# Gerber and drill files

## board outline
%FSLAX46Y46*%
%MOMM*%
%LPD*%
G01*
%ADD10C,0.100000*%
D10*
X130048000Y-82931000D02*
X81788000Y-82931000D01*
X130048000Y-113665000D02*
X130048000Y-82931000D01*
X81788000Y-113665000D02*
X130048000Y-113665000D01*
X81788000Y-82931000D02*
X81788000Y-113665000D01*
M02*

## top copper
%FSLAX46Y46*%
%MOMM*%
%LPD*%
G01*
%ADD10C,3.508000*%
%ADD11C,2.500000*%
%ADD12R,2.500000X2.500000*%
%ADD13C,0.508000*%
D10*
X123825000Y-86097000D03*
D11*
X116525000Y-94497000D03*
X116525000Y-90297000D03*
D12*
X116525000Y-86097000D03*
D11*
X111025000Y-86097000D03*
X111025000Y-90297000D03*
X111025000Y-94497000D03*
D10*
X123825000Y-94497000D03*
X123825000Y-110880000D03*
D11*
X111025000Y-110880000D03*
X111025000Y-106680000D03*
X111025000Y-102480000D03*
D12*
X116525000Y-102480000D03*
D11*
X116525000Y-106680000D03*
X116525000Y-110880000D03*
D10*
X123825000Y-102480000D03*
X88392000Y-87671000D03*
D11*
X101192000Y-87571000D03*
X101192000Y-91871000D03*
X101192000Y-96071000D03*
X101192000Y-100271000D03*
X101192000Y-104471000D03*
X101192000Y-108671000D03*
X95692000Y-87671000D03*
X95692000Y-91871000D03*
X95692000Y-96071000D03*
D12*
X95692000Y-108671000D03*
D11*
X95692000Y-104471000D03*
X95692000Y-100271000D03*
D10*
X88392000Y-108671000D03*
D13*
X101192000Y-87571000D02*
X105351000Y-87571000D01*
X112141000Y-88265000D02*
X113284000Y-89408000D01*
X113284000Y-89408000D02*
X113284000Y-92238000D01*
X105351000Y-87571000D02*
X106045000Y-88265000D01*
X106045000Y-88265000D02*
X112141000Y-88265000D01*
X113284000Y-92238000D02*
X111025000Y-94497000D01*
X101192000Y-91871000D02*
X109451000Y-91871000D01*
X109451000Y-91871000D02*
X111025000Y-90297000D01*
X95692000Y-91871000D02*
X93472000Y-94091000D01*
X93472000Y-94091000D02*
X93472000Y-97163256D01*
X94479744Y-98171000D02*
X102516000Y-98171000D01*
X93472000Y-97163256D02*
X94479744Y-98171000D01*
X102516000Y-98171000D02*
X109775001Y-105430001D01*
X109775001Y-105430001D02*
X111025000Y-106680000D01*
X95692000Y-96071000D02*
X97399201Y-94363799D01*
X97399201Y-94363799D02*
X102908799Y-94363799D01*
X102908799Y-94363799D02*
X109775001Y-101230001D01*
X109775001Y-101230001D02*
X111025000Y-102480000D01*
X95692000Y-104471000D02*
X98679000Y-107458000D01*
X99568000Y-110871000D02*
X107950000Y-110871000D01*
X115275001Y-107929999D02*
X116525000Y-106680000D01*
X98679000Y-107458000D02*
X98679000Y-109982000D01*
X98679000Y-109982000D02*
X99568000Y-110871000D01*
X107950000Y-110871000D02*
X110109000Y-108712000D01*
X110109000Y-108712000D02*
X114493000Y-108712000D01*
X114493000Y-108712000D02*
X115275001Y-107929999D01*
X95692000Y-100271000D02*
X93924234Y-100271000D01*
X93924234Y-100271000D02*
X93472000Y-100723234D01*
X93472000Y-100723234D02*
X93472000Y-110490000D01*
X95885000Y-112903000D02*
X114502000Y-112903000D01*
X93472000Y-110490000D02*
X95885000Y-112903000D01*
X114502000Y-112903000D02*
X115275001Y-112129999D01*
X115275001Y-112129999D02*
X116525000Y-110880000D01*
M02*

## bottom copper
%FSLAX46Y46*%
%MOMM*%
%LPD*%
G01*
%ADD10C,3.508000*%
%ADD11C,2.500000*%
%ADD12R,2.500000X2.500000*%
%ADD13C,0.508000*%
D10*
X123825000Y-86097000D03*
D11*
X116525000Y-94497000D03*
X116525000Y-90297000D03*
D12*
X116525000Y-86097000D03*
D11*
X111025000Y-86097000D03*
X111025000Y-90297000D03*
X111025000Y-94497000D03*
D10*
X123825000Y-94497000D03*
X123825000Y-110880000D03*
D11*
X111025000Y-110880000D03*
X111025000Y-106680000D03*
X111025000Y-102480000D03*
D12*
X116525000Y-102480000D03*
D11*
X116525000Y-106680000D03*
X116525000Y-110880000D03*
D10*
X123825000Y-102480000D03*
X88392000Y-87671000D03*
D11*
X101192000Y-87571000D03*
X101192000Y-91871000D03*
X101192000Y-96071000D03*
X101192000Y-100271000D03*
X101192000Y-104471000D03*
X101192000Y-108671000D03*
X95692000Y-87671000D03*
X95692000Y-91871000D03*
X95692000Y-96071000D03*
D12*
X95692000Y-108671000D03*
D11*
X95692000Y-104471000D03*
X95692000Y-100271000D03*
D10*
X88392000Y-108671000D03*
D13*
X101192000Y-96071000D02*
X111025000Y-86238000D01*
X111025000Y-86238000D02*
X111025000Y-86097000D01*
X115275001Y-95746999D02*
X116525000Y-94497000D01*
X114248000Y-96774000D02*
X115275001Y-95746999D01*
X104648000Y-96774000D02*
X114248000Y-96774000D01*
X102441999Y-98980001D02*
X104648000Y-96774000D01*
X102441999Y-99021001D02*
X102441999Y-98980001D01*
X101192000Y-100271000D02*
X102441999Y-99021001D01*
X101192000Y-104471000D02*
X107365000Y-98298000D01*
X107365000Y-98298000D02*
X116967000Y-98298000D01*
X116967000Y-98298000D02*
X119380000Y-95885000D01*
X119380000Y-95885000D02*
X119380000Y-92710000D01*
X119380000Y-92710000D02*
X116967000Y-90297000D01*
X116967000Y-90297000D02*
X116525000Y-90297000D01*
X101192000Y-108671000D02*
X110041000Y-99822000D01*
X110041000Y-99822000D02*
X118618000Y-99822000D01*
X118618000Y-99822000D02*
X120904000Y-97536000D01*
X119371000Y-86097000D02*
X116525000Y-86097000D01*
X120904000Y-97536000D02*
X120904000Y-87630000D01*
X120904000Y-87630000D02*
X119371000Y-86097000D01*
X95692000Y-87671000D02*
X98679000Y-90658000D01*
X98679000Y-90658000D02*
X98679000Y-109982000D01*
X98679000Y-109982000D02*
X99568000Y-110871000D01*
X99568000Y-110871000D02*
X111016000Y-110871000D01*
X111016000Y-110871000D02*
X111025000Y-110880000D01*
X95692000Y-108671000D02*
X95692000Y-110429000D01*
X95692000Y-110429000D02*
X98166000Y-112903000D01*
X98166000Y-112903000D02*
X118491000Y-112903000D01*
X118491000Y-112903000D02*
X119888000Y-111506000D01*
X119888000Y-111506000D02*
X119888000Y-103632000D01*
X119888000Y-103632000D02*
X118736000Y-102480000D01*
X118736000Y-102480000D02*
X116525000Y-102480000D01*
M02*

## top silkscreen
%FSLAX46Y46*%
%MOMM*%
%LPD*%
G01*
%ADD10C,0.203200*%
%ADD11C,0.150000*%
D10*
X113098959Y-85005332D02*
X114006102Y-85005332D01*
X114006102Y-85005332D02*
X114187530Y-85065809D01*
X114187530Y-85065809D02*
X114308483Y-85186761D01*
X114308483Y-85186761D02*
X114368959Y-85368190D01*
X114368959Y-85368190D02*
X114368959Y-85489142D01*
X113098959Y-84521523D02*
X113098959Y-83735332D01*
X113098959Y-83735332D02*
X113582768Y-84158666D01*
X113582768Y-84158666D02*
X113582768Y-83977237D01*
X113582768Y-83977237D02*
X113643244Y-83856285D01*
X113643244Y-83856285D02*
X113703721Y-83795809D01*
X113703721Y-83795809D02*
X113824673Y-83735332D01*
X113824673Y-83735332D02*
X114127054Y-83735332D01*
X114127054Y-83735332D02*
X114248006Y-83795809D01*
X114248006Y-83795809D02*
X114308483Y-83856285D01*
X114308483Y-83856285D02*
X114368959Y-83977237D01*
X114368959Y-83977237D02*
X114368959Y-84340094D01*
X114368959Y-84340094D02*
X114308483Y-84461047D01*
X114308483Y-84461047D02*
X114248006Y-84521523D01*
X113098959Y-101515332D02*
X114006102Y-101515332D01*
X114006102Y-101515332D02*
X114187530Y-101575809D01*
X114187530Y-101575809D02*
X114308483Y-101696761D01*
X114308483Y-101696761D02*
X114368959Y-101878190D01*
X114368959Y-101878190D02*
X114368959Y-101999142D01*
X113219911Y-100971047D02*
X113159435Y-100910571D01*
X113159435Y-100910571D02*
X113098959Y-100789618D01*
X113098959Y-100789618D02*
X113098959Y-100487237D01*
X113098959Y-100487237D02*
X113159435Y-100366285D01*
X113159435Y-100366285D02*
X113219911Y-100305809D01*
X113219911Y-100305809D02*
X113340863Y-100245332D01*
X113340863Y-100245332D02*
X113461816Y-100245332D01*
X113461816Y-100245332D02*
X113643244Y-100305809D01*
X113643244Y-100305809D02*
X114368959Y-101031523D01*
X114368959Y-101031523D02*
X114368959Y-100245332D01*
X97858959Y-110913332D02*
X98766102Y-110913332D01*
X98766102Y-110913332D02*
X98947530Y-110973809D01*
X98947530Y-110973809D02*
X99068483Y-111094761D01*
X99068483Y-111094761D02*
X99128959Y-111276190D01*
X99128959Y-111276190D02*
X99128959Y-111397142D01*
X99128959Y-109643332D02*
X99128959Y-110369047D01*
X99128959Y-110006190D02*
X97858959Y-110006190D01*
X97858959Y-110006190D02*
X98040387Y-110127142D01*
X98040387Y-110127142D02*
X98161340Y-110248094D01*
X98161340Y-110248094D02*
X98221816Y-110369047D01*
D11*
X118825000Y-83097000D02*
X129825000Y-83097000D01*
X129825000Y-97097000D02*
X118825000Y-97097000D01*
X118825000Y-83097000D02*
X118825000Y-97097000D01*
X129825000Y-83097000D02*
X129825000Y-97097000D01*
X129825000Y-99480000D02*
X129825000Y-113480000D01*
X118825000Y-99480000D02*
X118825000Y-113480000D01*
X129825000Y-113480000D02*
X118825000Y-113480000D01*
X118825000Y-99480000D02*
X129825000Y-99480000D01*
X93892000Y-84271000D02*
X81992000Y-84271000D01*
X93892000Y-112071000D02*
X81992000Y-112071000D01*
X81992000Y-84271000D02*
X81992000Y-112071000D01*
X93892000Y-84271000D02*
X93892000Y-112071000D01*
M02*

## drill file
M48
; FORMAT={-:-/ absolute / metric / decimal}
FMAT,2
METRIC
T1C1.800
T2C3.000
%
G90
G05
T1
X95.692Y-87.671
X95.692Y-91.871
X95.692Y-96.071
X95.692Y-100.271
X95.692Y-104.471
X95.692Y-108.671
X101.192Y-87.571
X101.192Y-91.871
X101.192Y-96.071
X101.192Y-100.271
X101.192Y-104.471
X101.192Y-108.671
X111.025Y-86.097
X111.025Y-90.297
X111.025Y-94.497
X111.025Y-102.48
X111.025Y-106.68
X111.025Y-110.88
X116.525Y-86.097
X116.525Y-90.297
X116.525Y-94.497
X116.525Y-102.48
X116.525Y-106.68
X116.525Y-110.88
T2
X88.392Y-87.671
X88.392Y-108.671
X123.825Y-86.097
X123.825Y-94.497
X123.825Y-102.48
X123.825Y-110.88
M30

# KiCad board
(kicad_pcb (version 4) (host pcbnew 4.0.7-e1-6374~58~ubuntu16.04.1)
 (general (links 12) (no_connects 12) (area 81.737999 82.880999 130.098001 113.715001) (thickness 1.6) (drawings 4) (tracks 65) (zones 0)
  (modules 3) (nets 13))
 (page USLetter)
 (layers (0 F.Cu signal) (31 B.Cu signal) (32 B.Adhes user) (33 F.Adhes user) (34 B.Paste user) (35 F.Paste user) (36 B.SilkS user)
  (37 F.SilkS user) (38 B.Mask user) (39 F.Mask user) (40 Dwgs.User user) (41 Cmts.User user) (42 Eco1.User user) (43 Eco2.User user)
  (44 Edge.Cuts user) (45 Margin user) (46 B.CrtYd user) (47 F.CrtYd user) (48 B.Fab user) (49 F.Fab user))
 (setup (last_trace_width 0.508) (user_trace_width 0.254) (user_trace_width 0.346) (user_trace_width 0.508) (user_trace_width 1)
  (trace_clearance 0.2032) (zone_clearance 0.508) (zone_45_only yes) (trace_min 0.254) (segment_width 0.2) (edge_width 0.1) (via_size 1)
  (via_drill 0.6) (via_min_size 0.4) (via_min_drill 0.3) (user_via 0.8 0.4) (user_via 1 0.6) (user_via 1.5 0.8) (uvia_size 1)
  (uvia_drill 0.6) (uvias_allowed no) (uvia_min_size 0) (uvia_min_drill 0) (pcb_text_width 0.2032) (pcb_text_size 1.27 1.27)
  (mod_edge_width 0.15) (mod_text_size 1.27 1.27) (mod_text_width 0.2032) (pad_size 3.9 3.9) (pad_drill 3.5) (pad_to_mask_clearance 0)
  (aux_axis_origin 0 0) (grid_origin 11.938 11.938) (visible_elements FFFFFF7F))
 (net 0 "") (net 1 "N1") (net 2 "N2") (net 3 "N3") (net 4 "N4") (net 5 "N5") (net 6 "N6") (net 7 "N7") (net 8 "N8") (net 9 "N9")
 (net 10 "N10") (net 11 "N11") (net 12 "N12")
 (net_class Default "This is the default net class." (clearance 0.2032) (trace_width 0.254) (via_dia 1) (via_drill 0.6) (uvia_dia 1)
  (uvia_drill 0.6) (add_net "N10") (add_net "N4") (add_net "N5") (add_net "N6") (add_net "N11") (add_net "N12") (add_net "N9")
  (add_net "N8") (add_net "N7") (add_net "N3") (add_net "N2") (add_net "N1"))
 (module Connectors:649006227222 (layer F.Cu) (at 123.825 90.297 90)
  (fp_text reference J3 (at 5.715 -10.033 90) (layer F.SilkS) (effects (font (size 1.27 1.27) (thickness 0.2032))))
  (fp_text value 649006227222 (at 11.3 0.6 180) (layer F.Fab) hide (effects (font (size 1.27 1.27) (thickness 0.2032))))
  (fp_line (start 7.2 -5) (end 7.2 6) (layer F.SilkS) (width 0.15))
  (fp_line (start -6.8 6) (end -6.8 -5) (layer F.SilkS) (width 0.15))
  (fp_line (start 7.2 -5) (end -6.8 -5) (layer F.SilkS) (width 0.15))
  (fp_line (start 7.2 6) (end -6.8 6) (layer F.SilkS) (width 0.15))
  (pad 7 thru_hole circle (at 4.2 0 90) (size 3.508 3.508) (drill 3) (layers *.Cu *.Mask))
  (pad 3 thru_hole circle (at -4.2 -7.3 90) (size 2.5 2.5) (drill 1.8) (layers *.Cu *.Mask) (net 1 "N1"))
  (pad 2 thru_hole circle (at 0 -7.3 90) (size 2.5 2.5) (drill 1.8) (layers *.Cu *.Mask) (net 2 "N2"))
  (pad 1 thru_hole rect (at 4.2 -7.3 90) (size 2.5 2.5) (drill 1.8) (layers *.Cu *.Mask) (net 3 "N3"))
  (pad 4 thru_hole circle (at 4.2 -12.8 90) (size 2.5 2.5) (drill 1.8) (layers *.Cu *.Mask) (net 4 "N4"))
  (pad 5 thru_hole circle (at 0 -12.8 90) (size 2.5 2.5) (drill 1.8) (layers *.Cu *.Mask) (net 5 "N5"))
  (pad 6 thru_hole circle (at -4.2 -12.8 90) (size 2.5 2.5) (drill 1.8) (layers *.Cu *.Mask) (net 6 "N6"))
  (pad 8 thru_hole circle (at -4.2 0 90) (size 3.508 3.508) (drill 3) (layers *.Cu *.Mask)))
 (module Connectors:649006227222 (layer F.Cu) (at 123.825 106.68 90)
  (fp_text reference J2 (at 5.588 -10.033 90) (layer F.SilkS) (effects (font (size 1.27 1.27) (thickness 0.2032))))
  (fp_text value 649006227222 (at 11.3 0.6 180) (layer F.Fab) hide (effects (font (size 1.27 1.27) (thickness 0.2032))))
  (fp_line (start 7.2 6) (end -6.8 6) (layer F.SilkS) (width 0.15))
  (fp_line (start 7.2 -5) (end -6.8 -5) (layer F.SilkS) (width 0.15))
  (fp_line (start -6.8 6) (end -6.8 -5) (layer F.SilkS) (width 0.15))
  (fp_line (start 7.2 -5) (end 7.2 6) (layer F.SilkS) (width 0.15))
  (pad 8 thru_hole circle (at -4.2 0 90) (size 3.508 3.508) (drill 3) (layers *.Cu *.Mask))
  (pad 6 thru_hole circle (at -4.2 -12.8 90) (size 2.5 2.5) (drill 1.8) (layers *.Cu *.Mask) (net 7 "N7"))
  (pad 5 thru_hole circle (at 0 -12.8 90) (size 2.5 2.5) (drill 1.8) (layers *.Cu *.Mask) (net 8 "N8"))
  (pad 4 thru_hole circle (at 4.2 -12.8 90) (size 2.5 2.5) (drill 1.8) (layers *.Cu *.Mask) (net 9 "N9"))
  (pad 1 thru_hole rect (at 4.2 -7.3 90) (size 2.5 2.5) (drill 1.8) (layers *.Cu *.Mask) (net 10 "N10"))
  (pad 2 thru_hole circle (at 0 -7.3 90) (size 2.5 2.5) (drill 1.8) (layers *.Cu *.Mask) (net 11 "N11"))
  (pad 3 thru_hole circle (at -4.2 -7.3 90) (size 2.5 2.5) (drill 1.8) (layers *.Cu *.Mask) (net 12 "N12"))
  (pad 7 thru_hole circle (at 4.2 0 90) (size 3.508 3.508) (drill 3) (layers *.Cu *.Mask)))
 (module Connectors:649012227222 (layer F.Cu) (at 88.392 98.171 270)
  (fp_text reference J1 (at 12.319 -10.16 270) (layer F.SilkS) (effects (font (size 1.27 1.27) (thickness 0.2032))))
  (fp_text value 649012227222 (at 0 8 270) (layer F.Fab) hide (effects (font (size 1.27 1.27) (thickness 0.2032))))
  (fp_line (start -13.9 -5.5) (end -13.9 6.4) (layer F.SilkS) (width 0.15))
  (fp_line (start 13.9 -5.5) (end 13.9 6.4) (layer F.SilkS) (width 0.15))
  (fp_line (start -13.9 6.4) (end 13.9 6.4) (layer F.SilkS) (width 0.15))
  (fp_line (start -13.9 -5.5) (end 13.9 -5.5) (layer F.SilkS) (width 0.15))
  (pad 14 thru_hole circle (at -10.5 0 270) (size 3.508 3.508) (drill 3) (layers *.Cu *.Mask))
  (pad 12 thru_hole circle (at -10.6 -12.8 270) (size 2.5 2.5) (drill 1.8) (layers *.Cu *.Mask) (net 6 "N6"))
  (pad 11 thru_hole circle (at -6.3 -12.8 270) (size 2.5 2.5) (drill 1.8) (layers *.Cu *.Mask) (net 5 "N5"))
  (pad 10 thru_hole circle (at -2.1 -12.8 270) (size 2.5 2.5) (drill 1.8) (layers *.Cu *.Mask) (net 4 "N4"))
  (pad 9 thru_hole circle (at 2.1 -12.8 270) (size 2.5 2.5) (drill 1.8) (layers *.Cu *.Mask) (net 1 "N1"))
  (pad 8 thru_hole circle (at 6.3 -12.8 270) (size 2.5 2.5) (drill 1.8) (layers *.Cu *.Mask) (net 2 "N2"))
  (pad 7 thru_hole circle (at 10.5 -12.8 270) (size 2.5 2.5) (drill 1.8) (layers *.Cu *.Mask) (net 3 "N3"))
  (pad 6 thru_hole circle (at -10.5 -7.3 270) (size 2.5 2.5) (drill 1.8) (layers *.Cu *.Mask) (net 7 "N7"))
  (pad 5 thru_hole circle (at -6.3 -7.3 270) (size 2.5 2.5) (drill 1.8) (layers *.Cu *.Mask) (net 8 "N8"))
  (pad 4 thru_hole circle (at -2.1 -7.3 270) (size 2.5 2.5) (drill 1.8) (layers *.Cu *.Mask) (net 9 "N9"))
  (pad 1 thru_hole rect (at 10.5 -7.3 270) (size 2.5 2.5) (drill 1.8) (layers *.Cu *.Mask) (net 10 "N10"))
  (pad 2 thru_hole circle (at 6.3 -7.3 270) (size 2.5 2.5) (drill 1.8) (layers *.Cu *.Mask) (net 11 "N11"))
  (pad 3 thru_hole circle (at 2.1 -7.3 270) (size 2.5 2.5) (drill 1.8) (layers *.Cu *.Mask) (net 12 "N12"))
  (pad 13 thru_hole circle (at 10.5 0 270) (size 3.508 3.508) (drill 3) (layers *.Cu *.Mask)))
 (gr_line (start 130.048 82.931) (end 81.788 82.931) (layer Edge.Cuts) (width 0.1))
 (gr_line (start 130.048 113.665) (end 130.048 82.931) (layer Edge.Cuts) (width 0.1))
 (gr_line (start 81.788 113.665) (end 130.048 113.665) (layer Edge.Cuts) (width 0.1))
 (gr_line (start 81.788 82.931) (end 81.788 113.665) (layer Edge.Cuts) (width 0.1))
 (segment (start 101.192 87.571) (end 105.351 87.571) (width 0.508) (layer F.Cu) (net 6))
 (segment (start 112.141 88.265) (end 113.284 89.408) (width 0.508) (layer F.Cu) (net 6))
 (segment (start 113.284 89.408) (end 113.284 92.238) (width 0.508) (layer F.Cu) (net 6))
 (segment (start 105.351 87.571) (end 106.045 88.265) (width 0.508) (layer F.Cu) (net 6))
 (segment (start 106.045 88.265) (end 112.141 88.265) (width 0.508) (layer F.Cu) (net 6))
 (segment (start 113.284 92.238) (end 111.025 94.497) (width 0.508) (layer F.Cu) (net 6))
 (segment (start 101.192 91.871) (end 109.451 91.871) (width 0.508) (layer F.Cu) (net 5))
 (segment (start 109.451 91.871) (end 111.025 90.297) (width 0.508) (layer F.Cu) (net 5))
 (segment (start 101.192 96.071) (end 111.025 86.238) (width 0.508) (layer B.Cu) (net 4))
 (segment (start 111.025 86.238) (end 111.025 86.097) (width 0.508) (layer B.Cu) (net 4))
 (segment (start 115.275001 95.746999) (end 116.525 94.497) (width 0.508) (layer B.Cu) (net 1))
 (segment (start 114.248 96.774) (end 115.275001 95.746999) (width 0.508) (layer B.Cu) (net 1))
 (segment (start 104.648 96.774) (end 114.248 96.774) (width 0.508) (layer B.Cu) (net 1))
 (segment (start 102.441999 98.980001) (end 104.648 96.774) (width 0.508) (layer B.Cu) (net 1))
 (segment (start 102.441999 99.021001) (end 102.441999 98.980001) (width 0.508) (layer B.Cu) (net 1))
 (segment (start 101.192 100.271) (end 102.441999 99.021001) (width 0.508) (layer B.Cu) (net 1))
 (segment (start 101.192 104.471) (end 107.365 98.298) (width 0.508) (layer B.Cu) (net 2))
 (segment (start 107.365 98.298) (end 116.967 98.298) (width 0.508) (layer B.Cu) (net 2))
 (segment (start 116.967 98.298) (end 119.38 95.885) (width 0.508) (layer B.Cu) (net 2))
 (segment (start 119.38 95.885) (end 119.38 92.71) (width 0.508) (layer B.Cu) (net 2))
 (segment (start 119.38 92.71) (end 116.967 90.297) (width 0.508) (layer B.Cu) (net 2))
 (segment (start 116.967 90.297) (end 116.525 90.297) (width 0.508) (layer B.Cu) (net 2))
 (segment (start 101.192 108.671) (end 110.041 99.822) (width 0.508) (layer B.Cu) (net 3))
 (segment (start 110.041 99.822) (end 118.618 99.822) (width 0.508) (layer B.Cu) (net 3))
 (segment (start 118.618 99.822) (end 120.904 97.536) (width 0.508) (layer B.Cu) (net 3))
 (segment (start 119.371 86.097) (end 116.525 86.097) (width 0.508) (layer B.Cu) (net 3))
 (segment (start 120.904 97.536) (end 120.904 87.63) (width 0.508) (layer B.Cu) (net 3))
 (segment (start 120.904 87.63) (end 119.371 86.097) (width 0.508) (layer B.Cu) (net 3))
 (segment (start 95.692 87.671) (end 98.679 90.658) (width 0.508) (layer B.Cu) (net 7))
 (segment (start 98.679 90.658) (end 98.679 109.982) (width 0.508) (layer B.Cu) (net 7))
 (segment (start 98.679 109.982) (end 99.568 110.871) (width 0.508) (layer B.Cu) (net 7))
 (segment (start 99.568 110.871) (end 111.016 110.871) (width 0.508) (layer B.Cu) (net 7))
 (segment (start 111.016 110.871) (end 111.025 110.88) (width 0.508) (layer B.Cu) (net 7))
 (segment (start 95.692 91.871) (end 93.472 94.091) (width 0.508) (layer F.Cu) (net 8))
 (segment (start 93.472 94.091) (end 93.472 97.163256) (width 0.508) (layer F.Cu) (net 8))
 (segment (start 94.479744 98.171) (end 102.516 98.171) (width 0.508) (layer F.Cu) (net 8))
 (segment (start 93.472 97.163256) (end 94.479744 98.171) (width 0.508) (layer F.Cu) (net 8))
 (segment (start 102.516 98.171) (end 109.775001 105.430001) (width 0.508) (layer F.Cu) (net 8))
 (segment (start 109.775001 105.430001) (end 111.025 106.68) (width 0.508) (layer F.Cu) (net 8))
 (segment (start 95.692 96.071) (end 97.399201 94.363799) (width 0.508) (layer F.Cu) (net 9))
 (segment (start 97.399201 94.363799) (end 102.908799 94.363799) (width 0.508) (layer F.Cu) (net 9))
 (segment (start 102.908799 94.363799) (end 109.775001 101.230001) (width 0.508) (layer F.Cu) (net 9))
 (segment (start 109.775001 101.230001) (end 111.025 102.48) (width 0.508) (layer F.Cu) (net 9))
 (segment (start 95.692 108.671) (end 95.692 110.429) (width 0.508) (layer B.Cu) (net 10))
 (segment (start 95.692 110.429) (end 98.166 112.903) (width 0.508) (layer B.Cu) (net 10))
 (segment (start 98.166 112.903) (end 118.491 112.903) (width 0.508) (layer B.Cu) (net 10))
 (segment (start 118.491 112.903) (end 119.888 111.506) (width 0.508) (layer B.Cu) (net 10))
 (segment (start 119.888 111.506) (end 119.888 103.632) (width 0.508) (layer B.Cu) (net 10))
 (segment (start 119.888 103.632) (end 118.736 102.48) (width 0.508) (layer B.Cu) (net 10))
 (segment (start 118.736 102.48) (end 116.525 102.48) (width 0.508) (layer B.Cu) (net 10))
 (segment (start 95.692 104.471) (end 98.679 107.458) (width 0.508) (layer F.Cu) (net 11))
 (segment (start 99.568 110.871) (end 107.95 110.871) (width 0.508) (layer F.Cu) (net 11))
 (segment (start 115.275001 107.929999) (end 116.525 106.68) (width 0.508) (layer F.Cu) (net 11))
 (segment (start 98.679 107.458) (end 98.679 109.982) (width 0.508) (layer F.Cu) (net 11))
 (segment (start 98.679 109.982) (end 99.568 110.871) (width 0.508) (layer F.Cu) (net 11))
 (segment (start 107.95 110.871) (end 110.109 108.712) (width 0.508) (layer F.Cu) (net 11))
 (segment (start 110.109 108.712) (end 114.493 108.712) (width 0.508) (layer F.Cu) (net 11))
 (segment (start 114.493 108.712) (end 115.275001 107.929999) (width 0.508) (layer F.Cu) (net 11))
 (segment (start 95.692 100.271) (end 93.924234 100.271) (width 0.508) (layer F.Cu) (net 12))
 (segment (start 93.924234 100.271) (end 93.472 100.723234) (width 0.508) (layer F.Cu) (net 12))
 (segment (start 93.472 100.723234) (end 93.472 110.49) (width 0.508) (layer F.Cu) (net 12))
 (segment (start 95.885 112.903) (end 114.502 112.903) (width 0.508) (layer F.Cu) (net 12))
 (segment (start 93.472 110.49) (end 95.885 112.903) (width 0.508) (layer F.Cu) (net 12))
 (segment (start 114.502 112.903) (end 115.275001 112.129999) (width 0.508) (layer F.Cu) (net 12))
 (segment (start 115.275001 112.129999) (end 116.525 110.88) (width 0.508) (layer F.Cu) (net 12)))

